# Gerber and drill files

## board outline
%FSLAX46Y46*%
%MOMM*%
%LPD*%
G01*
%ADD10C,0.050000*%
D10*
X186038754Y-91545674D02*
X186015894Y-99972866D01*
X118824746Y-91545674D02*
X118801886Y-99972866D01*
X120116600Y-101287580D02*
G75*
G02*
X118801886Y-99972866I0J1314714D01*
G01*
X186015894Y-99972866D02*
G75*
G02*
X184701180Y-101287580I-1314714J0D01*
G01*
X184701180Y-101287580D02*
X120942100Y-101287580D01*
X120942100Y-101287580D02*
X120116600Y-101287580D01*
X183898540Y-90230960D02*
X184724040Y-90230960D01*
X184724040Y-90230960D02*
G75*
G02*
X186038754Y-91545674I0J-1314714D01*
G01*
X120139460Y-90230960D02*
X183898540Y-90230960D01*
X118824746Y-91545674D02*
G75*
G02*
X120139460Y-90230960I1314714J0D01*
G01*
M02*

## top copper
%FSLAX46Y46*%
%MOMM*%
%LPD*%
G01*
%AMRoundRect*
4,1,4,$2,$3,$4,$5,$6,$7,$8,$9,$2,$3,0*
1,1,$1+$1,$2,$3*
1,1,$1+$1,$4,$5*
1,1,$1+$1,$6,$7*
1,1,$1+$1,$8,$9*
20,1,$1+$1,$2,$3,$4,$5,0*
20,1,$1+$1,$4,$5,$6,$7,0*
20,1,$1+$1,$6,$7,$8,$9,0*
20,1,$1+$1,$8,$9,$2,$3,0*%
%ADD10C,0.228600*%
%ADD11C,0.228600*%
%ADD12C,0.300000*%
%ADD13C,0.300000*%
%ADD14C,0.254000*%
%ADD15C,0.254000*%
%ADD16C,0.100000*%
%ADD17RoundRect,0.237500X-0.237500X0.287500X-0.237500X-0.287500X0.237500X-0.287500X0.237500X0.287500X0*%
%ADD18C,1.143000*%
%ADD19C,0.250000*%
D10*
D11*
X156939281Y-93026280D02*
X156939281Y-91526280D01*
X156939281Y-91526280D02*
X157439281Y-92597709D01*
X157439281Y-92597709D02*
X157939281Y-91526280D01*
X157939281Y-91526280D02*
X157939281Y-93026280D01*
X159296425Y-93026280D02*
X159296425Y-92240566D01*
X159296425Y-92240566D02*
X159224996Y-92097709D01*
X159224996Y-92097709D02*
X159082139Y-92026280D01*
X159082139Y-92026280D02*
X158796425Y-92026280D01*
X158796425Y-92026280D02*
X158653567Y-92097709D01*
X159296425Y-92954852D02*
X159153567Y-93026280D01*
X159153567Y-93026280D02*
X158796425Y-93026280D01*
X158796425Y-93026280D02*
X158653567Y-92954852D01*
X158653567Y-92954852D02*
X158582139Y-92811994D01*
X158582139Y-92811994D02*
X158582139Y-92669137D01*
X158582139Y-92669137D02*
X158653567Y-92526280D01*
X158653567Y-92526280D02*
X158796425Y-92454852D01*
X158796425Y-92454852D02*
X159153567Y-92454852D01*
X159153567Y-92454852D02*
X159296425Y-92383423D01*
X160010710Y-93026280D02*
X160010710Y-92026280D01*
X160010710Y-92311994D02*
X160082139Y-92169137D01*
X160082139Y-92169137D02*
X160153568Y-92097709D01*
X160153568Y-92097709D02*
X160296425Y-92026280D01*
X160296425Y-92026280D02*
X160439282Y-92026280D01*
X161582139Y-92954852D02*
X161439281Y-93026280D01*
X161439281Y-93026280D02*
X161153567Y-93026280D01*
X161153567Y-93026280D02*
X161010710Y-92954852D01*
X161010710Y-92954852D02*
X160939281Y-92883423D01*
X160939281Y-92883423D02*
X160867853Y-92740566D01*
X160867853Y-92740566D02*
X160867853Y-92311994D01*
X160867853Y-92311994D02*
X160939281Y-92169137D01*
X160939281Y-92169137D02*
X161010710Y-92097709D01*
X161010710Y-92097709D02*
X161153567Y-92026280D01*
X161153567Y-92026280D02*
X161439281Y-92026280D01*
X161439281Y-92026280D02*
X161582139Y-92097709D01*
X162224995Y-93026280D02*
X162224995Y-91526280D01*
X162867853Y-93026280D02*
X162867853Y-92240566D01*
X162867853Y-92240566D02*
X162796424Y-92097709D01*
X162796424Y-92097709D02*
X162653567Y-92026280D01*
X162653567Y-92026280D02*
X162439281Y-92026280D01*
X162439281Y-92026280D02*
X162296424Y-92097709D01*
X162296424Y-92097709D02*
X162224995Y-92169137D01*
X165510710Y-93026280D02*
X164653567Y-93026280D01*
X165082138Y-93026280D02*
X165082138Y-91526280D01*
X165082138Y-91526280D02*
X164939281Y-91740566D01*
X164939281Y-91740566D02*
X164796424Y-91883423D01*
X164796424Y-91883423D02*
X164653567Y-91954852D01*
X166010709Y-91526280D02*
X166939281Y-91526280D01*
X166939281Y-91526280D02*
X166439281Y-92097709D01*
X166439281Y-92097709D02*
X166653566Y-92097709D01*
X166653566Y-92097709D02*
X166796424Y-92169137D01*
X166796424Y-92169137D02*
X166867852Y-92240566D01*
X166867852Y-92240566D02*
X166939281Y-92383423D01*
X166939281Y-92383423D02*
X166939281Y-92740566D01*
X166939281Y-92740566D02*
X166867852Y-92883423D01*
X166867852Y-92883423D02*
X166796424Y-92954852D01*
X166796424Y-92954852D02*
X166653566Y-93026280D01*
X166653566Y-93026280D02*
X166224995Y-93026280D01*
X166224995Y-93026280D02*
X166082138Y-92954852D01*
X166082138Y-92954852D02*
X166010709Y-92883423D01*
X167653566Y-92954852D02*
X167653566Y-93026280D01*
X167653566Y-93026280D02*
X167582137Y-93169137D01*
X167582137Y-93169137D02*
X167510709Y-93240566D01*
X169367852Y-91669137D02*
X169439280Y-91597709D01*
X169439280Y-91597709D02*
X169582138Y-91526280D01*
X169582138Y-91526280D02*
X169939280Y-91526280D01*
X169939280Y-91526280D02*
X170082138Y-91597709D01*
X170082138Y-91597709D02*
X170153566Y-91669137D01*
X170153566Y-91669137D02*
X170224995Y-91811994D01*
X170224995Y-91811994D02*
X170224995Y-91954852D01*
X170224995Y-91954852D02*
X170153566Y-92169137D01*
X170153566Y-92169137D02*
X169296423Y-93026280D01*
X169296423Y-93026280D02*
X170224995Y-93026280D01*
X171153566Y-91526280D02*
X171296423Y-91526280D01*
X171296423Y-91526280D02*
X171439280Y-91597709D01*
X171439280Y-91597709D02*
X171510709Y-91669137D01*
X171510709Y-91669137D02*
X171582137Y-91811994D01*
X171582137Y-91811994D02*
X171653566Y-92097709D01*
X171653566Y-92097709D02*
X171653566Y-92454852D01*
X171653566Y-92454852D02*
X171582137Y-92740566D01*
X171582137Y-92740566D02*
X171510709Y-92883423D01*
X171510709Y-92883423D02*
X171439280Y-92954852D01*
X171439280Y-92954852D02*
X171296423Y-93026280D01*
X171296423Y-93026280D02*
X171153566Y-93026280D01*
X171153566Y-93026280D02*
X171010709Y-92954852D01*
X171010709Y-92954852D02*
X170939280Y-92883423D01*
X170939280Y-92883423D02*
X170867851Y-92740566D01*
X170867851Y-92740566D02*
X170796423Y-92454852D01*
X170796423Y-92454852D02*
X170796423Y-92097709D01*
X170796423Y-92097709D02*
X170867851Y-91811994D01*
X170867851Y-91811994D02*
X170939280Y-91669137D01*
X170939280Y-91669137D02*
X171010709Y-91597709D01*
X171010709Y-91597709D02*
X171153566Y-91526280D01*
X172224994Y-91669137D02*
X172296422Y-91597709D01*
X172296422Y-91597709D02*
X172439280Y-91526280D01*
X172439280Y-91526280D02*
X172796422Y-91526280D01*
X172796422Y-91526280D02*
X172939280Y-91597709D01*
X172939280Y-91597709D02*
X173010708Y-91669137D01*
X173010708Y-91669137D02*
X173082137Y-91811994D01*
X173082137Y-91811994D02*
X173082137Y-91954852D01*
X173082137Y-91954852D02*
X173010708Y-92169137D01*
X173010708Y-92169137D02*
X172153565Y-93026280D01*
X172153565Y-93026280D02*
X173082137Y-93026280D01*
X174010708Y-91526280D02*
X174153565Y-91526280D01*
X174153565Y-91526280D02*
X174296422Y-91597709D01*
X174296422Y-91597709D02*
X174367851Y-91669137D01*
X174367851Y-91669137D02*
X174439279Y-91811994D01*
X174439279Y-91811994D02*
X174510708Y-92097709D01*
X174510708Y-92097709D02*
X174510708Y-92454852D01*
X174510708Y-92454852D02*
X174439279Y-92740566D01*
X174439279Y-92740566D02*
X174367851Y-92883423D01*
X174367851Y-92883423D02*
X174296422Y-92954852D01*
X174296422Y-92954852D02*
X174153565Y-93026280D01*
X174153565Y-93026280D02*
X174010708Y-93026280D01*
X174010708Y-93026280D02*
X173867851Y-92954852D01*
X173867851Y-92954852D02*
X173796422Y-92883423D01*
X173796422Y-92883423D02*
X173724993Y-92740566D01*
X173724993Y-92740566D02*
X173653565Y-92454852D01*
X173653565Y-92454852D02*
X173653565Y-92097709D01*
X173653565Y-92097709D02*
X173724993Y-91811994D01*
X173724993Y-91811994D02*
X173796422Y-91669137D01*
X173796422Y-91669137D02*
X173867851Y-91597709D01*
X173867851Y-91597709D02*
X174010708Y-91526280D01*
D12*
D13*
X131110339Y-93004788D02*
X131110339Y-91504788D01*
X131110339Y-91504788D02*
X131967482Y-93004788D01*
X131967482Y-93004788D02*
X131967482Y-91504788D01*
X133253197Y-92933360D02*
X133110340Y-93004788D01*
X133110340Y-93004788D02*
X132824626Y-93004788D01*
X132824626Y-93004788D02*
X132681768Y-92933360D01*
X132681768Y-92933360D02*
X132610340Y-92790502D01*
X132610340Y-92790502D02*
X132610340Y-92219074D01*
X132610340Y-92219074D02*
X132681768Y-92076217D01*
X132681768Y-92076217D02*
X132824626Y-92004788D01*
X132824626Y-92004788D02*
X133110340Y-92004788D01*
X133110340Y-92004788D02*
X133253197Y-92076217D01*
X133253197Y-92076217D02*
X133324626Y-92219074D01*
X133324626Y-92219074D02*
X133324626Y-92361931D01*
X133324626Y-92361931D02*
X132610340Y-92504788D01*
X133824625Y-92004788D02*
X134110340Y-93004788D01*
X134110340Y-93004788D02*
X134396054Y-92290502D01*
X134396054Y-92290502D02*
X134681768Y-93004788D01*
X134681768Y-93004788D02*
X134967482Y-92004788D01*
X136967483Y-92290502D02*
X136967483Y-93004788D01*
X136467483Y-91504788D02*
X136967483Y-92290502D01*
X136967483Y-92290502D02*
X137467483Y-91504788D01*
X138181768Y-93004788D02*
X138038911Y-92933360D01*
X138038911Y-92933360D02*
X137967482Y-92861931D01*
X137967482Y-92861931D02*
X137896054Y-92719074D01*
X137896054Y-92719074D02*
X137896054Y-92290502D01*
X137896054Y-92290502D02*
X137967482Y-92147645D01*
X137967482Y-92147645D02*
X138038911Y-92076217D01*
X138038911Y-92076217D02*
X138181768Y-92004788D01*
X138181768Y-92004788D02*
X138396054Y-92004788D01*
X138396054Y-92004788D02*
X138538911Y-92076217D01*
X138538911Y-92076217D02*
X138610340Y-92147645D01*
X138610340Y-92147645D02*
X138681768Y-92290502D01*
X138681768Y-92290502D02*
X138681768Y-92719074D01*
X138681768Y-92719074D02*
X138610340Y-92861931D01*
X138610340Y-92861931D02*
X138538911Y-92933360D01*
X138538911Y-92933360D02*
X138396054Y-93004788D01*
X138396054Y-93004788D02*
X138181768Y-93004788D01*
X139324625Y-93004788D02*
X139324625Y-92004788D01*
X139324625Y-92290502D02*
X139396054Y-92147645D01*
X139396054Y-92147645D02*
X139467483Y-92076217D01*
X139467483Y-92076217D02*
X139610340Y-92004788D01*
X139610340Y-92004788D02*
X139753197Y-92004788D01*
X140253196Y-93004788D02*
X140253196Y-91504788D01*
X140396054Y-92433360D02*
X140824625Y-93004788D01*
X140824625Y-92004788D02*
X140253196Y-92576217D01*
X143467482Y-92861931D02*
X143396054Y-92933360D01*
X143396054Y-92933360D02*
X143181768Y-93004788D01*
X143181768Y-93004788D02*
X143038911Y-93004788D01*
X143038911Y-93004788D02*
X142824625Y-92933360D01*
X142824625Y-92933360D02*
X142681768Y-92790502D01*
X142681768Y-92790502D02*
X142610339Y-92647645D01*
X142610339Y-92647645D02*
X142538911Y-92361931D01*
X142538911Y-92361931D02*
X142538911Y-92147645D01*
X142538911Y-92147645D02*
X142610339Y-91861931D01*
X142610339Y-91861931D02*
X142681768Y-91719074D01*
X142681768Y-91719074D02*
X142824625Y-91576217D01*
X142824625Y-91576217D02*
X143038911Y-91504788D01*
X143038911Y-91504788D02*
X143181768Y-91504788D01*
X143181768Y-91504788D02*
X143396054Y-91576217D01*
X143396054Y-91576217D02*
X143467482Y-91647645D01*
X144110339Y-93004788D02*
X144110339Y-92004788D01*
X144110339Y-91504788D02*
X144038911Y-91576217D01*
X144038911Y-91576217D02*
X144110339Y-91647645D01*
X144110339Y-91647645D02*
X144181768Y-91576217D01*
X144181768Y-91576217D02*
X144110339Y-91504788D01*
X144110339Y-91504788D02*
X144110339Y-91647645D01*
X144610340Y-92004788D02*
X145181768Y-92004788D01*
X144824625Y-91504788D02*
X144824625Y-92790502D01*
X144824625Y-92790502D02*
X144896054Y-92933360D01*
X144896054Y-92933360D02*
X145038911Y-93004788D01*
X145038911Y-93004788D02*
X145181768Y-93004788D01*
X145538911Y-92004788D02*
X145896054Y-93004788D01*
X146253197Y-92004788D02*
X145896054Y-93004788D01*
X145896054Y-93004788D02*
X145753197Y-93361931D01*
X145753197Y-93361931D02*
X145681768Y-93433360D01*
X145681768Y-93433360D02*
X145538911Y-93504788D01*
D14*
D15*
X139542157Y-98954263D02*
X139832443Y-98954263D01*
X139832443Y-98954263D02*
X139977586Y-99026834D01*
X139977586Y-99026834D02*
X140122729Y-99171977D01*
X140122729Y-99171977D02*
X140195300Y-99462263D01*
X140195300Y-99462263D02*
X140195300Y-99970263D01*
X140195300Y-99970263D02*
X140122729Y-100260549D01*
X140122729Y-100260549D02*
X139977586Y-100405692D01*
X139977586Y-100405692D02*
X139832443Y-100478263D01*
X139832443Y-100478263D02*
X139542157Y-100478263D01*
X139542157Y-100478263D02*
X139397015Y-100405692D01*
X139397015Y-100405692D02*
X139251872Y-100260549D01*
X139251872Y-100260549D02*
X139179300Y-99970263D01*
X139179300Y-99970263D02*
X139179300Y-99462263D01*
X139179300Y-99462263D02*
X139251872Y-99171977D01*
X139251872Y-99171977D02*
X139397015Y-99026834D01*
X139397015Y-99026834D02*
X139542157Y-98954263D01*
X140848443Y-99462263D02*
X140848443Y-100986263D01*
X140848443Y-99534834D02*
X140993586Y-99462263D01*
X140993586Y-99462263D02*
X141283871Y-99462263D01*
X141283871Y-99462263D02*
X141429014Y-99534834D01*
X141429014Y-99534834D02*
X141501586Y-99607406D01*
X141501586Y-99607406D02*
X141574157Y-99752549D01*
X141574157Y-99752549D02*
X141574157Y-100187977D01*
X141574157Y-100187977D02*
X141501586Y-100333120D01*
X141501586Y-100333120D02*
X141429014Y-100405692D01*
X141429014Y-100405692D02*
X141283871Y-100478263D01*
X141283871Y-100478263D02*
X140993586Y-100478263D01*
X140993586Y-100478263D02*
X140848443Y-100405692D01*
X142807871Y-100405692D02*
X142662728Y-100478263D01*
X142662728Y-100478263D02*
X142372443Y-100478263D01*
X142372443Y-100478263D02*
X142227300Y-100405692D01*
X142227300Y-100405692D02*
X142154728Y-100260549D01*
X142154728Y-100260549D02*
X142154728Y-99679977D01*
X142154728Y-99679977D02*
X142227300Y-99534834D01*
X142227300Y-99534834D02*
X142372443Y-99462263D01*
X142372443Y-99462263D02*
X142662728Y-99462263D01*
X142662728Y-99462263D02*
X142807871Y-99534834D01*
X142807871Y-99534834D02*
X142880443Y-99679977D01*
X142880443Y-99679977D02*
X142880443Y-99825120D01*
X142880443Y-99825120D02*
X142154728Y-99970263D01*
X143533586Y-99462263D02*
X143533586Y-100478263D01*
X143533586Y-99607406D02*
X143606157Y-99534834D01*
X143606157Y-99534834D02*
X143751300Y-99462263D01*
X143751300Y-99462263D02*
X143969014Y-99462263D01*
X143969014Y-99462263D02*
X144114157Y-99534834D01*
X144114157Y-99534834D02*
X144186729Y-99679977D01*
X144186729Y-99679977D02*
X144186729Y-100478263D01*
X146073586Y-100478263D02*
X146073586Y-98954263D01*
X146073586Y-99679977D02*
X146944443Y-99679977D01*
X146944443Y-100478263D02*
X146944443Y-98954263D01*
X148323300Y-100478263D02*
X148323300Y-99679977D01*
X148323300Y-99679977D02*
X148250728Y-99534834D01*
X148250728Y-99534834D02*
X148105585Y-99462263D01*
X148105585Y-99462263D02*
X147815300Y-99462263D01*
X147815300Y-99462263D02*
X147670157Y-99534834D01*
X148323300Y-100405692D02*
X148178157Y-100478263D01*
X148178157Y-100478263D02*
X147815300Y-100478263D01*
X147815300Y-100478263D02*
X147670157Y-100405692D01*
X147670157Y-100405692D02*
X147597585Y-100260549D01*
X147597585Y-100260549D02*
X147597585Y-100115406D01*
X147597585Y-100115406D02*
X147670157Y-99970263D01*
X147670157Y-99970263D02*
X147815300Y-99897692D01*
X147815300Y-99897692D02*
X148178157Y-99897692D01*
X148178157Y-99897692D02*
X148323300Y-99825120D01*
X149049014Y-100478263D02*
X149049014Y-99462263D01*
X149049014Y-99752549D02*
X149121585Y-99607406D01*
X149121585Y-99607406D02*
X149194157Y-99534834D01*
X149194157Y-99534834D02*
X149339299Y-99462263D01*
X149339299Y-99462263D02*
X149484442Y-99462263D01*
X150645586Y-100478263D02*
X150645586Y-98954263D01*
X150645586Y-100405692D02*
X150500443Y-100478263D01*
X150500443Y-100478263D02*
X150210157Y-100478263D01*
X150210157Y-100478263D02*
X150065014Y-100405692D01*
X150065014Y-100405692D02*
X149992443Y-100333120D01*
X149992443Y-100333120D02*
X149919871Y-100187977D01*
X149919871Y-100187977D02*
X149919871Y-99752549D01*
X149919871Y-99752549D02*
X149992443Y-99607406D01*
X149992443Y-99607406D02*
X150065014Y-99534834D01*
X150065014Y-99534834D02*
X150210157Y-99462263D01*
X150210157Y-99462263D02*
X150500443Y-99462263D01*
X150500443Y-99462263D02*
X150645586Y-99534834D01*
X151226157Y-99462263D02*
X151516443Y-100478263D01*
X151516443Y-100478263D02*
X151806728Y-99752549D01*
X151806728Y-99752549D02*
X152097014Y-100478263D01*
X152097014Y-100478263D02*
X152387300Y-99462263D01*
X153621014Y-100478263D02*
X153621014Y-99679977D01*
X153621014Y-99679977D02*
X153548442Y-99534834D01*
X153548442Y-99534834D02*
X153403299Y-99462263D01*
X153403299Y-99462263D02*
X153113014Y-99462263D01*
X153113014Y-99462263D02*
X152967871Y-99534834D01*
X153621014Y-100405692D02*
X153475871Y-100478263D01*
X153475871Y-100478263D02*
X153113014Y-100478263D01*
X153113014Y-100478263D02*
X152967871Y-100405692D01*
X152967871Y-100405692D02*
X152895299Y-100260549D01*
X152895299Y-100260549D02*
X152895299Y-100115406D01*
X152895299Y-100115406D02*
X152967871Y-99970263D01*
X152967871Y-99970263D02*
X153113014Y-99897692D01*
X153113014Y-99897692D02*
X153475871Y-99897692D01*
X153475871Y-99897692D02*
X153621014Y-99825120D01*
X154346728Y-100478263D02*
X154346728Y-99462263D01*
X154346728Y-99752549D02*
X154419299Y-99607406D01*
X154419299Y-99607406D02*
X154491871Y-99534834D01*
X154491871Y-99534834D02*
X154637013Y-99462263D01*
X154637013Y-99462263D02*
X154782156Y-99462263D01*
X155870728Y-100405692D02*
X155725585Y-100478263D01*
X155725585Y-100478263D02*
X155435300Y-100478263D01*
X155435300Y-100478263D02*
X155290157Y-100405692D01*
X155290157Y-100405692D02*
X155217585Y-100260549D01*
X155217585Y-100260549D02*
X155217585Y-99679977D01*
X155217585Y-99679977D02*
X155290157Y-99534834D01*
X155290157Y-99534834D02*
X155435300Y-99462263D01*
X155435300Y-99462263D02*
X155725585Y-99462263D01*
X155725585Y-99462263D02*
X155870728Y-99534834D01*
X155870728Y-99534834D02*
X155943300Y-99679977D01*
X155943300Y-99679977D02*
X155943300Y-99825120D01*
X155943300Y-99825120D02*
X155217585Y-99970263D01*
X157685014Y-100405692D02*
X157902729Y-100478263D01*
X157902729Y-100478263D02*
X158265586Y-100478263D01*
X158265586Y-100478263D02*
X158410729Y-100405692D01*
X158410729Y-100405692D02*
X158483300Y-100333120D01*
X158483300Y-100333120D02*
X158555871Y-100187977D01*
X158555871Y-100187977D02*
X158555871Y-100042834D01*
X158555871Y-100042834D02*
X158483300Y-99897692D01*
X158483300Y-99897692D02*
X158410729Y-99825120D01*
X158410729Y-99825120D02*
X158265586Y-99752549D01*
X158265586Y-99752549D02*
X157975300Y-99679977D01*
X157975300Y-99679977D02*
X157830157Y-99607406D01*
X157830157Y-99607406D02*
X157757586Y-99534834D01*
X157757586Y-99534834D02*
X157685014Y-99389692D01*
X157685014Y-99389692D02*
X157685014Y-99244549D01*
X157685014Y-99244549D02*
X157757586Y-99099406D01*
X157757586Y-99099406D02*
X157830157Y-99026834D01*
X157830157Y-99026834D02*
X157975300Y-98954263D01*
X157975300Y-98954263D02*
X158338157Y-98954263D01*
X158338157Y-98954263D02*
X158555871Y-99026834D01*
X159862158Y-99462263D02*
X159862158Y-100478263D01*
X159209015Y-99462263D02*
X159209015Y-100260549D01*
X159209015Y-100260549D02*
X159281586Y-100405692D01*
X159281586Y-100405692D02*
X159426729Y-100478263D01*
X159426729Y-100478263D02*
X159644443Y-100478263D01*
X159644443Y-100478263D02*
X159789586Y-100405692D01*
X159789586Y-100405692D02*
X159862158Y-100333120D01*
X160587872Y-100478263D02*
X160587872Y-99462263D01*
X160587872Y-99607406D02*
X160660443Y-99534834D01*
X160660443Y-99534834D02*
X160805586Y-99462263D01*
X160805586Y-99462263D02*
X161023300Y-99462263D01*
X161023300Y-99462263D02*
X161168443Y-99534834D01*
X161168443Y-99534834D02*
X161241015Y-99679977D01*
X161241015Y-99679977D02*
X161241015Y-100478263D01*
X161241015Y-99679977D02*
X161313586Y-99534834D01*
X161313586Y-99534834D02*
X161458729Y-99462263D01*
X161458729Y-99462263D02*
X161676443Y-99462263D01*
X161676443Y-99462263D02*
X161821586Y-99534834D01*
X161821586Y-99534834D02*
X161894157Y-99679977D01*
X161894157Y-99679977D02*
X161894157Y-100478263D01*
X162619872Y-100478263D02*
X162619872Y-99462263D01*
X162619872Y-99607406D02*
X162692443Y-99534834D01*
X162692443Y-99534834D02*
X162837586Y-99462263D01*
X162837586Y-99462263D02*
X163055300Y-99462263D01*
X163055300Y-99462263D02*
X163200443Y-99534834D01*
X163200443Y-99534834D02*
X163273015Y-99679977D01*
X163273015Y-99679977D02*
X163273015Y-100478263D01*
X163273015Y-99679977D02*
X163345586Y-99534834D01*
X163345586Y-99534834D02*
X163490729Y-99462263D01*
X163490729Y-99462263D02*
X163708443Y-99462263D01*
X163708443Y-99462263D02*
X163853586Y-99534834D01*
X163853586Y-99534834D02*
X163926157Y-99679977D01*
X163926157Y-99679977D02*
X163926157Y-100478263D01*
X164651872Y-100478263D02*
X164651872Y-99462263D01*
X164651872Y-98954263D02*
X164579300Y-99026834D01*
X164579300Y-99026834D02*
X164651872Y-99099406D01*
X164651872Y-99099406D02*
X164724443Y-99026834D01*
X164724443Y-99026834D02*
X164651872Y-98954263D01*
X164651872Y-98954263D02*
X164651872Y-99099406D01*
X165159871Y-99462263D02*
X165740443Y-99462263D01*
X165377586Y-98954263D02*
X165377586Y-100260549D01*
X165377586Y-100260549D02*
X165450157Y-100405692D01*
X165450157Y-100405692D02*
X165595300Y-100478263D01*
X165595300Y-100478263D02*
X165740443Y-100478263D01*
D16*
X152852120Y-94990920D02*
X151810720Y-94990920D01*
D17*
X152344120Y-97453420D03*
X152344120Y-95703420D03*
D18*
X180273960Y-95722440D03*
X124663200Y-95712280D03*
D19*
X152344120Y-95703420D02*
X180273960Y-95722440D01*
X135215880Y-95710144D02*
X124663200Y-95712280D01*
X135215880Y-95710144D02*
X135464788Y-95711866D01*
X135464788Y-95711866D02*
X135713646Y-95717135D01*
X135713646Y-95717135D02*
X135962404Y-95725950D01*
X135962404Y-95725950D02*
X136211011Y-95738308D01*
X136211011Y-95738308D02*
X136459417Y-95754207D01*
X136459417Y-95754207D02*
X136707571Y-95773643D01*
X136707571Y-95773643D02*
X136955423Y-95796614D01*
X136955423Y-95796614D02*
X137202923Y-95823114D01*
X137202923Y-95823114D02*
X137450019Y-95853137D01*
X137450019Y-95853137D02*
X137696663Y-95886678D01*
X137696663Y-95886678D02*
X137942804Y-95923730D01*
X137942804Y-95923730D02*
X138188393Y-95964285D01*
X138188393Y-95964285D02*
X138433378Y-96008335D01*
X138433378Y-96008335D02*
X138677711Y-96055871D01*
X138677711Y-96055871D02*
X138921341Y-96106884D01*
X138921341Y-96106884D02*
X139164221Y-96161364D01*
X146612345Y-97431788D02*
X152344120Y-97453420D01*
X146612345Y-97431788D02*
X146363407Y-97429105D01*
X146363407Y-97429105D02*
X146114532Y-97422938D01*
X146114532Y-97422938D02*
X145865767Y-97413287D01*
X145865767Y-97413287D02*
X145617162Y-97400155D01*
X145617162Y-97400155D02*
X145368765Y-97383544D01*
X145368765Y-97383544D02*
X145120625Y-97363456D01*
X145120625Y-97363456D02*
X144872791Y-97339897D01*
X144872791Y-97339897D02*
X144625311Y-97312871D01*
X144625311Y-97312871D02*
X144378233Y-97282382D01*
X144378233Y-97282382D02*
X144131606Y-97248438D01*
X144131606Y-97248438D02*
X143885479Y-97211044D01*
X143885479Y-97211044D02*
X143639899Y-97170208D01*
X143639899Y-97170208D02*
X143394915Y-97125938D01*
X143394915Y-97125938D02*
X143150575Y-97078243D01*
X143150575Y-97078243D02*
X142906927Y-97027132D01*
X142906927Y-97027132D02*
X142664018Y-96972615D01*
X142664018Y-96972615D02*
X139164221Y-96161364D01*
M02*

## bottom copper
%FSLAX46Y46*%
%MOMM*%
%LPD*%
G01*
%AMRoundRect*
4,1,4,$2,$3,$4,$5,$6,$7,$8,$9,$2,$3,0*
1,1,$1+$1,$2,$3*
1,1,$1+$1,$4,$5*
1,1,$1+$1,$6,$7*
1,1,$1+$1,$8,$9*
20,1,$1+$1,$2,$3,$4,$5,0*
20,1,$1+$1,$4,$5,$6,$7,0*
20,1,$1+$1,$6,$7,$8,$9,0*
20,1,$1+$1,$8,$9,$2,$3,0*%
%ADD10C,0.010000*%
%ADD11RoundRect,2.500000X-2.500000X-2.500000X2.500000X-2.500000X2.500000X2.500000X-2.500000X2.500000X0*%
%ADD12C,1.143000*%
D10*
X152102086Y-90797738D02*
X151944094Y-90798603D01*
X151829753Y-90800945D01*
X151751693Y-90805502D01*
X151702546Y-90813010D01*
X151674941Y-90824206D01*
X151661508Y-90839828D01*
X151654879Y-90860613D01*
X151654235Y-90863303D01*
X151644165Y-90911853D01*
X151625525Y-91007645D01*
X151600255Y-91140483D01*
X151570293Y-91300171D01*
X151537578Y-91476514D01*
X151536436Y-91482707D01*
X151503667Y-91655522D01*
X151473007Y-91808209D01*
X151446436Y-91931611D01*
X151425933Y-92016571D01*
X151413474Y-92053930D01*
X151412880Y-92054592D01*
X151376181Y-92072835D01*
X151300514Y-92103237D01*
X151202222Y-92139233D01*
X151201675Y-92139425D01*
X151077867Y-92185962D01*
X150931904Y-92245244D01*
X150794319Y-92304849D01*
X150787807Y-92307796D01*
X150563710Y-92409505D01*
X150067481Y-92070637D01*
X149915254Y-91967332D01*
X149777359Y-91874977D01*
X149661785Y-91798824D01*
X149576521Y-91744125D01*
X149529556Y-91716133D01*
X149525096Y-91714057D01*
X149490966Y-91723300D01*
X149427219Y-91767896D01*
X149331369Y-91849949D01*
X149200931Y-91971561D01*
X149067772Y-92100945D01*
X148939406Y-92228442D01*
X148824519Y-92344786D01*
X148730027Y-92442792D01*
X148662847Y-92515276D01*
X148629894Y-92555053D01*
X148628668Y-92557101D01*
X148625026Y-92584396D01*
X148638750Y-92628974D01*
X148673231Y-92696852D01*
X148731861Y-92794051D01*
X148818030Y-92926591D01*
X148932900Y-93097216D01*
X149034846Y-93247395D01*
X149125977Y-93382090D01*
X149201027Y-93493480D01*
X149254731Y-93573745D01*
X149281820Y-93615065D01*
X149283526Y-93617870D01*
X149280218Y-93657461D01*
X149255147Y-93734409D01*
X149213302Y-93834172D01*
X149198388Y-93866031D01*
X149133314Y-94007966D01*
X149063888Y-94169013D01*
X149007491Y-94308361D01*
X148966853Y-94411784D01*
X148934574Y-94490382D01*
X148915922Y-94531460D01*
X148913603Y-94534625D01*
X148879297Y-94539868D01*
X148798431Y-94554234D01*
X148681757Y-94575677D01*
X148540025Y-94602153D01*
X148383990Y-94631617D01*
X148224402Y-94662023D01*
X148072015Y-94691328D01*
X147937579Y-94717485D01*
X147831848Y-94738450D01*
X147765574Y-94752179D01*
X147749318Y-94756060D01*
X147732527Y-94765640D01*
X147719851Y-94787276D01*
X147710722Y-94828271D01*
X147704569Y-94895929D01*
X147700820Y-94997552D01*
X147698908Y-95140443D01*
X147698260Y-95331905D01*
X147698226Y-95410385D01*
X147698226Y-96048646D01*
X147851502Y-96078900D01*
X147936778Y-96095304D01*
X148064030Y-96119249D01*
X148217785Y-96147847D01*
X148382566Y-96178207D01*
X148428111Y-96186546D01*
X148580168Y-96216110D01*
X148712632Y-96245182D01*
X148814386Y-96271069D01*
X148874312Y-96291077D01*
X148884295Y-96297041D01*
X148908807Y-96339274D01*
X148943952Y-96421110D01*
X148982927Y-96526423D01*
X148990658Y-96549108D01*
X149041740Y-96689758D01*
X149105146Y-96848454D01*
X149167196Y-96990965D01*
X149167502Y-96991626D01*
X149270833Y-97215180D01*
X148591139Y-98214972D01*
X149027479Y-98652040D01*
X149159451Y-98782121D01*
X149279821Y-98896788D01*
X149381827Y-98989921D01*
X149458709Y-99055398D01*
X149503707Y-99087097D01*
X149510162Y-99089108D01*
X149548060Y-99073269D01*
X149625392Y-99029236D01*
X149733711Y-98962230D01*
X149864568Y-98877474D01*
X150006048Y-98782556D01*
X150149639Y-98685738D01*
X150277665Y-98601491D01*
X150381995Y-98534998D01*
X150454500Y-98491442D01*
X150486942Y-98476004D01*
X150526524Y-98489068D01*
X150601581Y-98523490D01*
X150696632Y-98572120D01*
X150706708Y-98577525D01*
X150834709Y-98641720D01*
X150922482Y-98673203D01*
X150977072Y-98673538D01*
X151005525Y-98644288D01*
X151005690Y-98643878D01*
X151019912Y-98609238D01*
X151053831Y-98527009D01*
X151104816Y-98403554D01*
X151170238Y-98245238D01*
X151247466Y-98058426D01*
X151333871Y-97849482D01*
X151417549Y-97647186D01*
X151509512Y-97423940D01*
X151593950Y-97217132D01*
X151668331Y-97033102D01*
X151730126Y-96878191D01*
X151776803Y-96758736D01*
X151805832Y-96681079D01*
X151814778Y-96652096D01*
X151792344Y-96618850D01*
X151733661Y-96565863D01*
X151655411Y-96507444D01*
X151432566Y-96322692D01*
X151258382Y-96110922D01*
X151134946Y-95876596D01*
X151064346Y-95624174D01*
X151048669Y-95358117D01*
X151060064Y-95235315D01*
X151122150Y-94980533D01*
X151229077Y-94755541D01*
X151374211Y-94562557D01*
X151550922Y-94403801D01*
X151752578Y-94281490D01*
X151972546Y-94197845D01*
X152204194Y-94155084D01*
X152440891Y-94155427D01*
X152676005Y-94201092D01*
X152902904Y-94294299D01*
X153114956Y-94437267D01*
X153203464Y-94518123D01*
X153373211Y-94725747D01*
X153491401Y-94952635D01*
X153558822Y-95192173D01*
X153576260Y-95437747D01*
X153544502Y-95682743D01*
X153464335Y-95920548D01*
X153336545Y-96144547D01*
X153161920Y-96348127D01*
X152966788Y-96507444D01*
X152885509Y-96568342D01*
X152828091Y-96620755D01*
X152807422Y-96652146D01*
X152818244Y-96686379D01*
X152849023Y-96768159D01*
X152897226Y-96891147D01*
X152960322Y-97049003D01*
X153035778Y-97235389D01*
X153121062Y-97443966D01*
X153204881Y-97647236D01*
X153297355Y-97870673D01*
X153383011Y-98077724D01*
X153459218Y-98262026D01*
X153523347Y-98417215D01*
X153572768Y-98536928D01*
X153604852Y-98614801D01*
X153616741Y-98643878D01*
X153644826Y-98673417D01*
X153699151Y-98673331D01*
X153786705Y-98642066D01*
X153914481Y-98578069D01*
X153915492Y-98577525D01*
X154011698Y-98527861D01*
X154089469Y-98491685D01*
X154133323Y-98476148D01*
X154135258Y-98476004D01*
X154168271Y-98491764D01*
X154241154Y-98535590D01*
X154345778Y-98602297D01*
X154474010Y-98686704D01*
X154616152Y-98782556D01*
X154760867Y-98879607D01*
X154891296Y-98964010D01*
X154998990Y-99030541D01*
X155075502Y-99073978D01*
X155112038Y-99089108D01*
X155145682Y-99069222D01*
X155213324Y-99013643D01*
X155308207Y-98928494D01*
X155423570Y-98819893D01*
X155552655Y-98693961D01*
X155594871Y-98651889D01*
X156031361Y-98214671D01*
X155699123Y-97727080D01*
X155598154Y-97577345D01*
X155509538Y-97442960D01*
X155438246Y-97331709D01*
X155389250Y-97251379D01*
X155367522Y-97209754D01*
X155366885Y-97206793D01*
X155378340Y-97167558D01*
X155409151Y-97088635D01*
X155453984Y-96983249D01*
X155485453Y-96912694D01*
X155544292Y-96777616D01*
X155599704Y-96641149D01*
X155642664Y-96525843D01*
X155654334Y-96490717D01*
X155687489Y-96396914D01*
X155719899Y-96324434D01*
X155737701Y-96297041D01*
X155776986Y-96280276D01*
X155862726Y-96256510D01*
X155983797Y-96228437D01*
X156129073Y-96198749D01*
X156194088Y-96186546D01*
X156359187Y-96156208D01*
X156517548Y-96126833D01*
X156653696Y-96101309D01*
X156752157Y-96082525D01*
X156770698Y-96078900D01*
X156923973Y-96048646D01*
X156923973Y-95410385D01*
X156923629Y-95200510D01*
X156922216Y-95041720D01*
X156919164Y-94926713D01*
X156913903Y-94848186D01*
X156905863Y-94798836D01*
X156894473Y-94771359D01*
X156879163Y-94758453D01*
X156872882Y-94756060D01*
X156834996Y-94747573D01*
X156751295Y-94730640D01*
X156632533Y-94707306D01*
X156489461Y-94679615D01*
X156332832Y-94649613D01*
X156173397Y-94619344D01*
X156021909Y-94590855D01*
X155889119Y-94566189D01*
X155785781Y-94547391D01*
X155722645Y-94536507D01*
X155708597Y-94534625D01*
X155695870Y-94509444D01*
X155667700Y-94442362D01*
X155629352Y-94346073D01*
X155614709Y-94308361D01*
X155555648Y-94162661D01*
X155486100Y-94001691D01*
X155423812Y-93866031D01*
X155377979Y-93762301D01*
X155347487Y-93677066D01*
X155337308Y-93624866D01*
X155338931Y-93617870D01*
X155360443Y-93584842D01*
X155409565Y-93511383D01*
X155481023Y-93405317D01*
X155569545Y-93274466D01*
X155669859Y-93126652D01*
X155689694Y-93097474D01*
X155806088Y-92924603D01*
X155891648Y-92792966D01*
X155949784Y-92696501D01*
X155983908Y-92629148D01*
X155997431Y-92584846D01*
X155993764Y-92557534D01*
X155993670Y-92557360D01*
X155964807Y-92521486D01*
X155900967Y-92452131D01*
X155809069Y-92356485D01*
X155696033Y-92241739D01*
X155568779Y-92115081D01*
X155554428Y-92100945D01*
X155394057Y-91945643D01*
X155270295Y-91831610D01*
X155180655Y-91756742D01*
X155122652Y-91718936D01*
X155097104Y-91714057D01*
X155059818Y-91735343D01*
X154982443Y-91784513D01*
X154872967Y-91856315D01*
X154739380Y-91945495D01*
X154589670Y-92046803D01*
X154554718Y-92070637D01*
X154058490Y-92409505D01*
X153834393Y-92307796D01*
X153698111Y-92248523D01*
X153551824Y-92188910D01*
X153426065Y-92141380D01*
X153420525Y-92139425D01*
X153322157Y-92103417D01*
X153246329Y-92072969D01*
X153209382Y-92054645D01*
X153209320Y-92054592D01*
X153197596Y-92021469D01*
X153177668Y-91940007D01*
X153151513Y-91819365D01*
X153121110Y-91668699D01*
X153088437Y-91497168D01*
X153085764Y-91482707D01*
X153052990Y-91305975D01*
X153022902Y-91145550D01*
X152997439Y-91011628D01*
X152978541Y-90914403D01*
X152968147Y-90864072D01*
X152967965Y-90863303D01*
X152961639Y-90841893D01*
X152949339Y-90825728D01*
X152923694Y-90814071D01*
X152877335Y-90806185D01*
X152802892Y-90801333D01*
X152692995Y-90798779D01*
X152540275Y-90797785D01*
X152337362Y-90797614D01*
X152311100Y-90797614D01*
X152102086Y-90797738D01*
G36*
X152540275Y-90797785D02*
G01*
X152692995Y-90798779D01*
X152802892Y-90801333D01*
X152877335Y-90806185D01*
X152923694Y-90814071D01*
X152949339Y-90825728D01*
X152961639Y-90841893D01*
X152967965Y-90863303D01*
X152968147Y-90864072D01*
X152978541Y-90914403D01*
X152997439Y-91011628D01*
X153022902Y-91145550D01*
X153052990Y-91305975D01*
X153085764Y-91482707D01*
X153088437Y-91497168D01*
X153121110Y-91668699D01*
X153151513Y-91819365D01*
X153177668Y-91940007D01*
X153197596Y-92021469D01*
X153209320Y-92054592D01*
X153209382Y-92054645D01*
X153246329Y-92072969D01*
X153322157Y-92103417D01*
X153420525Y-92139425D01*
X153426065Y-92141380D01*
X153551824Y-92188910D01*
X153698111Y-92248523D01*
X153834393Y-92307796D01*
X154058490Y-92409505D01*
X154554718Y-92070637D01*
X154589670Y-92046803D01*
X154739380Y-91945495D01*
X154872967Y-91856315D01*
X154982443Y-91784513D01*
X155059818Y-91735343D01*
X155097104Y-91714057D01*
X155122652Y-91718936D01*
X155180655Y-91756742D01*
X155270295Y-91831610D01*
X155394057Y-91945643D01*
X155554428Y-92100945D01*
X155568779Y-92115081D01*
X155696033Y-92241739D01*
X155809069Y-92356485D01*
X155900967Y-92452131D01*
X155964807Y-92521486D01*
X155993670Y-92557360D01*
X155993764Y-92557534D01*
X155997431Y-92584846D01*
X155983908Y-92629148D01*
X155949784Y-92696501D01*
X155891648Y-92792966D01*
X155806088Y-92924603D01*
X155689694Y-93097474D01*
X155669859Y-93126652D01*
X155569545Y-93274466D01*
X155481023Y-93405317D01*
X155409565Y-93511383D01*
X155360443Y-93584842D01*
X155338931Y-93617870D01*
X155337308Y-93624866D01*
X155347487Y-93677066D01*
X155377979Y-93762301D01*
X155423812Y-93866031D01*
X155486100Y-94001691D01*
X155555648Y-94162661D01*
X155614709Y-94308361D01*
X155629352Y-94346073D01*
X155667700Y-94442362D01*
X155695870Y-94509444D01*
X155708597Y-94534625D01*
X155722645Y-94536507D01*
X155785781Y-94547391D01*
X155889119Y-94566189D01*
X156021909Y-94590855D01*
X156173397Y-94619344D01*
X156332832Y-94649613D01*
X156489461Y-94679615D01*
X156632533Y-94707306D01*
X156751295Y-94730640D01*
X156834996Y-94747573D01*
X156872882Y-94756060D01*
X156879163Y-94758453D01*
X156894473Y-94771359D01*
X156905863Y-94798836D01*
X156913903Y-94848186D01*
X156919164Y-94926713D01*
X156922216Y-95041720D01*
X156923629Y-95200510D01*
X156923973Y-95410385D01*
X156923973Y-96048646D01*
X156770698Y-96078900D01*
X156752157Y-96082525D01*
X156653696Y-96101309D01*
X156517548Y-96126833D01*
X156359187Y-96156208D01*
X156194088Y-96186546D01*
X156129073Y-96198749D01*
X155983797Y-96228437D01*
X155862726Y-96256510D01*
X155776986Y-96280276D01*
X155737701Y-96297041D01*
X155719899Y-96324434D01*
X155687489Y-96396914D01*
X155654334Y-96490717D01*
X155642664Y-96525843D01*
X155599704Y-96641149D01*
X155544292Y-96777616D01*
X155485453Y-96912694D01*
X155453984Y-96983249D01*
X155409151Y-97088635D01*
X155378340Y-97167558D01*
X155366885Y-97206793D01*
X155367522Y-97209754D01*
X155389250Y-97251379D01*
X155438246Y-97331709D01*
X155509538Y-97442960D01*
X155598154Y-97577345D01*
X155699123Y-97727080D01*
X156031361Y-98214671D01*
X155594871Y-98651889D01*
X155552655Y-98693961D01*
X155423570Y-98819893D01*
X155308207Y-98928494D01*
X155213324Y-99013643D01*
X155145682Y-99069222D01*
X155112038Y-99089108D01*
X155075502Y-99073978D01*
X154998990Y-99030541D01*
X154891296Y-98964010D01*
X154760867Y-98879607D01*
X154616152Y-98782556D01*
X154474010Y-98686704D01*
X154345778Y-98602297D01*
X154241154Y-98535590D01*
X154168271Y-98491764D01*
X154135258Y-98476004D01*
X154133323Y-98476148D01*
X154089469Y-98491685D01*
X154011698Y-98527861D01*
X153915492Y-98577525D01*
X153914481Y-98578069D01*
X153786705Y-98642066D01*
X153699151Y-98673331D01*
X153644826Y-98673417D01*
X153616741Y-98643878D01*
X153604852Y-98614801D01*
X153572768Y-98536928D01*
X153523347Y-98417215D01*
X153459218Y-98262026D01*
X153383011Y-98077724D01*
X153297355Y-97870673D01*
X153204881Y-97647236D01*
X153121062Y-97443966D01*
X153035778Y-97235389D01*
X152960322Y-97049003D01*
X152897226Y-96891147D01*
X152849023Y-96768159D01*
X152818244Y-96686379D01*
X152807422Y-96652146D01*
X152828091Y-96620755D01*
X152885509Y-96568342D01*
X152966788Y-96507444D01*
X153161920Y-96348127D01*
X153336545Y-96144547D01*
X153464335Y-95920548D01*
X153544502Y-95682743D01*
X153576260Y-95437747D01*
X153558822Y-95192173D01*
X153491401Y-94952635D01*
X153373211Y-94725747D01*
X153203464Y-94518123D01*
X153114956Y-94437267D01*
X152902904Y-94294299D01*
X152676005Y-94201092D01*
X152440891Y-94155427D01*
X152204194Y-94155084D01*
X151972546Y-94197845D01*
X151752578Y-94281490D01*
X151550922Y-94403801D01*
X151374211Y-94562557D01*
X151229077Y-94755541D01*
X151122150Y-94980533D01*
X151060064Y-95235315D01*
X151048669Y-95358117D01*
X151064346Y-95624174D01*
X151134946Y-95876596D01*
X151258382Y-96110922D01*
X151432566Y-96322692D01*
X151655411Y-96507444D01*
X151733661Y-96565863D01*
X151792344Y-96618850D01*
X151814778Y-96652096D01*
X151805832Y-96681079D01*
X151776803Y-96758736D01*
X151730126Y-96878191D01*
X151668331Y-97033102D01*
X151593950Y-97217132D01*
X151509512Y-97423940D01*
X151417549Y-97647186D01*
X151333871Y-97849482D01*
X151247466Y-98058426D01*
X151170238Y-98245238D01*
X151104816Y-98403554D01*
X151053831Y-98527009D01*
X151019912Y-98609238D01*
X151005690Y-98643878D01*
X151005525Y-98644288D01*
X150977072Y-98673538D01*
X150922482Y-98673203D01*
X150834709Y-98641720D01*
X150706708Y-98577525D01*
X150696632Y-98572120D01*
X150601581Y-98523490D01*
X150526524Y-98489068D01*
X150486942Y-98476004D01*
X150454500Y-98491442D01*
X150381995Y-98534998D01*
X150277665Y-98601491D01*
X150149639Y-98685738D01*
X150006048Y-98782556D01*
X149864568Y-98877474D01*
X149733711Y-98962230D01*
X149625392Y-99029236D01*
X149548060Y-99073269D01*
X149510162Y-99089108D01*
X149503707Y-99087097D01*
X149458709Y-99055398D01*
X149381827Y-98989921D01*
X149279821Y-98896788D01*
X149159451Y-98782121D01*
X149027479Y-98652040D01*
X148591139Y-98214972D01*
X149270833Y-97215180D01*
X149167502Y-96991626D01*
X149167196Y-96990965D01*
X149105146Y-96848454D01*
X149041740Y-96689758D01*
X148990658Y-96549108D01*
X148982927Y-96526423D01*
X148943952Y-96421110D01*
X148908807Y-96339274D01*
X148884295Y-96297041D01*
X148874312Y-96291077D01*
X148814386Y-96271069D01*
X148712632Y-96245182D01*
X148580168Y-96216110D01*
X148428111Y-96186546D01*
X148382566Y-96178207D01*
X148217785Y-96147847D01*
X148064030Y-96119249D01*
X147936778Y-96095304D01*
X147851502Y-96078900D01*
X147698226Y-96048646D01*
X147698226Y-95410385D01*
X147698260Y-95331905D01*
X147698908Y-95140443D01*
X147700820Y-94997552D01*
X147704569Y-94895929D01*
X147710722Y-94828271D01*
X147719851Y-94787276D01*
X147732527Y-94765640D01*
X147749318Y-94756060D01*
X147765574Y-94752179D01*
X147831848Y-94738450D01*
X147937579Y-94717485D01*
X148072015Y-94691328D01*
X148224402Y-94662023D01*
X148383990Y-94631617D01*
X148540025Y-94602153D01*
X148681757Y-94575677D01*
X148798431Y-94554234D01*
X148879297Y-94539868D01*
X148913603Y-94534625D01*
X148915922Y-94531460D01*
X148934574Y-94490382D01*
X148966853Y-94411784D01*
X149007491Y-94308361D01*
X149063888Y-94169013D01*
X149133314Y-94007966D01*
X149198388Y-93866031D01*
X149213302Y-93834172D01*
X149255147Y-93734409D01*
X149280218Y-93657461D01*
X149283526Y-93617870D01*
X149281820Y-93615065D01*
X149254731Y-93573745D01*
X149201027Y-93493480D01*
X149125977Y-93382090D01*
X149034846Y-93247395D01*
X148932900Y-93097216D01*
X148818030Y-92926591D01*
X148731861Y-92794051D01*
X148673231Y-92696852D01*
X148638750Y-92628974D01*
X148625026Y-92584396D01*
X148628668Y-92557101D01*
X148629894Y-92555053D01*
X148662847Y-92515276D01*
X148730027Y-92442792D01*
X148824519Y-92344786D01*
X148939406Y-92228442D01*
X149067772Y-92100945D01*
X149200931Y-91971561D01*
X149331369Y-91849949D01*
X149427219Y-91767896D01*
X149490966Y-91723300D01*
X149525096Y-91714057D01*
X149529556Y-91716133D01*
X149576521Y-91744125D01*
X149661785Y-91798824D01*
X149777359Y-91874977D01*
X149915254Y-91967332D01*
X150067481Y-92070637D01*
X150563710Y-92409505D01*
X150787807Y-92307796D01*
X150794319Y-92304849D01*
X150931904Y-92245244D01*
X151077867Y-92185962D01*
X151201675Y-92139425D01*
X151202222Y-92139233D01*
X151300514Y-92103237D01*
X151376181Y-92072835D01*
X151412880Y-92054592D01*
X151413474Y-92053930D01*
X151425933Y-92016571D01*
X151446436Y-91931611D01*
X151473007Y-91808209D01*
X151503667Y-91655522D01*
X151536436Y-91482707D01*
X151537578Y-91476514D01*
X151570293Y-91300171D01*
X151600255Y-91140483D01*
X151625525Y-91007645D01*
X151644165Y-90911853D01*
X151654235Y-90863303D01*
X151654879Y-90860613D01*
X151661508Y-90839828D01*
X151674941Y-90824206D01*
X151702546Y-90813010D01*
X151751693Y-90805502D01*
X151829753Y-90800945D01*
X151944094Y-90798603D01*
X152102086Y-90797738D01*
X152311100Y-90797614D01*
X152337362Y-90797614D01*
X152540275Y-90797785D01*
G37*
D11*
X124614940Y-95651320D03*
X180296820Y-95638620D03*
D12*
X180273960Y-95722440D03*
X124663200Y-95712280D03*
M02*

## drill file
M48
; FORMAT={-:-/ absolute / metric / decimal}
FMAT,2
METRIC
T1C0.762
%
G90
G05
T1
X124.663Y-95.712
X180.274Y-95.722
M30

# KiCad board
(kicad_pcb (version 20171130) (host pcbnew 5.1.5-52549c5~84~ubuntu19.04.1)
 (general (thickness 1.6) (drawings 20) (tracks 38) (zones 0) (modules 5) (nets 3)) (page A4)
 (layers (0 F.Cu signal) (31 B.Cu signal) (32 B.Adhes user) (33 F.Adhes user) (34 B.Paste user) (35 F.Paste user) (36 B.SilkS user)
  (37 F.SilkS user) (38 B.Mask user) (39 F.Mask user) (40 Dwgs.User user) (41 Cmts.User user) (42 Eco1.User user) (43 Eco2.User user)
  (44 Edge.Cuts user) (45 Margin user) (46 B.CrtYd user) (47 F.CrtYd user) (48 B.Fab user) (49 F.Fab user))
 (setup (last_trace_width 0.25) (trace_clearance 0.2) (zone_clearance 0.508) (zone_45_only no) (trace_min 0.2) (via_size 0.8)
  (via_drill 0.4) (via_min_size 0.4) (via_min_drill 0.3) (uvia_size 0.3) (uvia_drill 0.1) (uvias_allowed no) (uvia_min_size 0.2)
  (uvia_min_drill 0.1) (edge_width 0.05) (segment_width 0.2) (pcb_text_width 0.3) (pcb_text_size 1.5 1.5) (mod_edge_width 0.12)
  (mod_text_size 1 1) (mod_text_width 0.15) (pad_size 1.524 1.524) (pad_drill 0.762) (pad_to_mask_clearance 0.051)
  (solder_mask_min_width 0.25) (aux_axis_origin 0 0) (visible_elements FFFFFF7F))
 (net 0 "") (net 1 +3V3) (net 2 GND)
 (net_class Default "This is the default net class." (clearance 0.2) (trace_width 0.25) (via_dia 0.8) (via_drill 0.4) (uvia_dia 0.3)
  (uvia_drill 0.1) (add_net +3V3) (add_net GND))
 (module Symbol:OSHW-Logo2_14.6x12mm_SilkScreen (layer B.Cu) (at 152.3111 96.34474 180)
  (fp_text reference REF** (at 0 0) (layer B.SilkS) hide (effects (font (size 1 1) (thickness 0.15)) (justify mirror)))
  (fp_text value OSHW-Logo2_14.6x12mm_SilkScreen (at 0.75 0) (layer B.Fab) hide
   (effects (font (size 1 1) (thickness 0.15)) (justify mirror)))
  (fp_poly
   (pts (xy 0.209014 5.547002) (xy 0.367006 5.546137) (xy 0.481347 5.543795) (xy 0.559407 5.539238) (xy 0.608554 5.53173)
    (xy 0.636159 5.520534) (xy 0.649592 5.504912) (xy 0.656221 5.484127) (xy 0.656865 5.481437) (xy 0.666935 5.432887)
    (xy 0.685575 5.337095) (xy 0.710845 5.204257) (xy 0.740807 5.044569) (xy 0.773522 4.868226) (xy 0.774664 4.862033)
    (xy 0.807433 4.689218) (xy 0.838093 4.536531) (xy 0.864664 4.413129) (xy 0.885167 4.328169) (xy 0.897626 4.29081) (xy 0.89822 4.290148)
    (xy 0.934919 4.271905) (xy 1.010586 4.241503) (xy 1.108878 4.205507) (xy 1.109425 4.205315) (xy 1.233233 4.158778)
    (xy 1.379196 4.099496) (xy 1.516781 4.039891) (xy 1.523293 4.036944) (xy 1.74739 3.935235) (xy 2.243619 4.274103) (xy 2.395846 4.377408)
    (xy 2.533741 4.469763) (xy 2.649315 4.545916) (xy 2.734579 4.600615) (xy 2.781544 4.628607) (xy 2.786004 4.630683) (xy 2.820134 4.62144)
    (xy 2.883881 4.576844) (xy 2.979731 4.494791) (xy 3.110169 4.373179) (xy 3.243328 4.243795) (xy 3.371694 4.116298)
    (xy 3.486581 3.999954) (xy 3.581073 3.901948) (xy 3.648253 3.829464) (xy 3.681206 3.789687) (xy 3.682432 3.787639)
    (xy 3.686074 3.760344) (xy 3.67235 3.715766) (xy 3.637869 3.647888) (xy 3.579239 3.550689) (xy 3.49307 3.418149) (xy 3.3782 3.247524)
    (xy 3.276254 3.097345) (xy 3.185123 2.96265) (xy 3.110073 2.85126) (xy 3.056369 2.770995) (xy 3.02928 2.729675) (xy 3.027574 2.72687)
    (xy 3.030882 2.687279) (xy 3.055953 2.610331) (xy 3.097798 2.510568) (xy 3.112712 2.478709) (xy 3.177786 2.336774)
    (xy 3.247212 2.175727) (xy 3.303609 2.036379) (xy 3.344247 1.932956) (xy 3.376526 1.854358) (xy 3.395178 1.81328) (xy 3.397497 1.810115)
    (xy 3.431803 1.804872) (xy 3.512669 1.790506) (xy 3.629343 1.769063) (xy 3.771075 1.742587) (xy 3.92711 1.713123) (xy 4.086698 1.682717)
    (xy 4.239085 1.653412) (xy 4.373521 1.627255) (xy 4.479252 1.60629) (xy 4.545526 1.592561) (xy 4.561782 1.58868) (xy 4.578573 1.5791)
    (xy 4.591249 1.557464) (xy 4.600378 1.516469) (xy 4.606531 1.448811) (xy 4.61028 1.347188) (xy 4.612192 1.204297) (xy 4.61284 1.012835)
    (xy 4.612874 0.934355) (xy 4.612874 0.296094) (xy 4.459598 0.26584) (xy 4.374322 0.249436) (xy 4.24707 0.225491) (xy 4.093315 0.196893)
    (xy 3.928534 0.166533) (xy 3.882989 0.158194) (xy 3.730932 0.12863) (xy 3.598468 0.099558) (xy 3.496714 0.073671) (xy 3.436788 0.053663)
    (xy 3.426805 0.047699) (xy 3.402293 0.005466) (xy 3.367148 -0.07637) (xy 3.328173 -0.181683) (xy 3.320442 -0.204368)
    (xy 3.26936 -0.345018) (xy 3.205954 -0.503714) (xy 3.143904 -0.646225) (xy 3.143598 -0.646886) (xy 3.040267 -0.87044)
    (xy 3.719961 -1.870232) (xy 3.283621 -2.3073) (xy 3.151649 -2.437381) (xy 3.031279 -2.552048) (xy 2.929273 -2.645181)
    (xy 2.852391 -2.710658) (xy 2.807393 -2.742357) (xy 2.800938 -2.744368) (xy 2.76304 -2.728529) (xy 2.685708 -2.684496)
    (xy 2.577389 -2.61749) (xy 2.446532 -2.532734) (xy 2.305052 -2.437816) (xy 2.161461 -2.340998) (xy 2.033435 -2.256751)
    (xy 1.929105 -2.190258) (xy 1.8566 -2.146702) (xy 1.824158 -2.131264) (xy 1.784576 -2.144328) (xy 1.709519 -2.17875)
    (xy 1.614468 -2.22738) (xy 1.604392 -2.232785) (xy 1.476391 -2.29698) (xy 1.388618 -2.328463) (xy 1.334028 -2.328798)
    (xy 1.305575 -2.299548) (xy 1.30541 -2.299138) (xy 1.291188 -2.264498) (xy 1.257269 -2.182269) (xy 1.206284 -2.058814)
    (xy 1.140862 -1.900498) (xy 1.063634 -1.713686) (xy 0.977229 -1.504742) (xy 0.893551 -1.302446) (xy 0.801588 -1.0792)
    (xy 0.71715 -0.872392) (xy 0.642769 -0.688362) (xy 0.580974 -0.533451) (xy 0.534297 -0.413996) (xy 0.505268 -0.336339)
    (xy 0.496322 -0.307356) (xy 0.518756 -0.27411) (xy 0.577439 -0.221123) (xy 0.655689 -0.162704) (xy 0.878534 0.022048)
    (xy 1.052718 0.233818) (xy 1.176154 0.468144) (xy 1.246754 0.720566) (xy 1.262431 0.986623) (xy 1.251036 1.109425) (xy 1.18895 1.364207)
    (xy 1.082023 1.589199) (xy 0.936889 1.782183) (xy 0.760178 1.940939) (xy 0.558522 2.06325) (xy 0.338554 2.146895) (xy 0.106906 2.189656)
    (xy -0.129791 2.189313) (xy -0.364905 2.143648) (xy -0.591804 2.050441) (xy -0.803856 1.907473) (xy -0.892364 1.826617)
    (xy -1.062111 1.618993) (xy -1.180301 1.392105) (xy -1.247722 1.152567) (xy -1.26516 0.906993) (xy -1.233402 0.661997)
    (xy -1.153235 0.424192) (xy -1.025445 0.200193) (xy -0.85082 -0.003387) (xy -0.655688 -0.162704) (xy -0.574409 -0.223602)
    (xy -0.516991 -0.276015) (xy -0.496322 -0.307406) (xy -0.507144 -0.341639) (xy -0.537923 -0.423419) (xy -0.586126 -0.546407)
    (xy -0.649222 -0.704263) (xy -0.724678 -0.890649) (xy -0.809962 -1.099226) (xy -0.893781 -1.302496) (xy -0.986255 -1.525933)
    (xy -1.071911 -1.732984) (xy -1.148118 -1.917286) (xy -1.212247 -2.072475) (xy -1.261668 -2.192188) (xy -1.293752 -2.270061)
    (xy -1.305641 -2.299138) (xy -1.333726 -2.328677) (xy -1.388051 -2.328591) (xy -1.475605 -2.297326) (xy -1.603381 -2.233329)
    (xy -1.604392 -2.232785) (xy -1.700598 -2.183121) (xy -1.778369 -2.146945) (xy -1.822223 -2.131408) (xy -1.824158 -2.131264)
    (xy -1.857171 -2.147024) (xy -1.930054 -2.19085) (xy -2.034678 -2.257557) (xy -2.16291 -2.341964) (xy -2.305052 -2.437816)
    (xy -2.449767 -2.534867) (xy -2.580196 -2.61927) (xy -2.68789 -2.685801) (xy -2.764402 -2.729238) (xy -2.800938 -2.744368)
    (xy -2.834582 -2.724482) (xy -2.902224 -2.668903) (xy -2.997107 -2.583754) (xy -3.11247 -2.475153) (xy -3.241555 -2.349221)
    (xy -3.283771 -2.307149) (xy -3.720261 -1.869931) (xy -3.388023 -1.38234) (xy -3.287054 -1.232605) (xy -3.198438 -1.09822)
    (xy -3.127146 -0.986969) (xy -3.07815 -0.906639) (xy -3.056422 -0.865014) (xy -3.055785 -0.862053) (xy -3.06724 -0.822818)
    (xy -3.098051 -0.743895) (xy -3.142884 -0.638509) (xy -3.174353 -0.567954) (xy -3.233192 -0.432876) (xy -3.288604 -0.296409)
    (xy -3.331564 -0.181103) (xy -3.343234 -0.145977) (xy -3.376389 -0.052174) (xy -3.408799 0.020306) (xy -3.426601 0.047699)
    (xy -3.465886 0.064464) (xy -3.551626 0.08823) (xy -3.672697 0.116303) (xy -3.817973 0.145991) (xy -3.882988 0.158194)
    (xy -4.048087 0.188532) (xy -4.206448 0.217907) (xy -4.342596 0.243431) (xy -4.441057 0.262215) (xy -4.459598 0.26584)
    (xy -4.612873 0.296094) (xy -4.612873 0.934355) (xy -4.612529 1.14423) (xy -4.611116 1.30302) (xy -4.608064 1.418027)
    (xy -4.602803 1.496554) (xy -4.594763 1.545904) (xy -4.583373 1.573381) (xy -4.568063 1.586287) (xy -4.561782 1.58868)
    (xy -4.523896 1.597167) (xy -4.440195 1.6141) (xy -4.321433 1.637434) (xy -4.178361 1.665125) (xy -4.021732 1.695127)
    (xy -3.862297 1.725396) (xy -3.710809 1.753885) (xy -3.578019 1.778551) (xy -3.474681 1.797349) (xy -3.411545 1.808233)
    (xy -3.397497 1.810115) (xy -3.38477 1.835296) (xy -3.3566 1.902378) (xy -3.318252 1.998667) (xy -3.303609 2.036379)
    (xy -3.244548 2.182079) (xy -3.175 2.343049) (xy -3.112712 2.478709) (xy -3.066879 2.582439) (xy -3.036387 2.667674)
    (xy -3.026208 2.719874) (xy -3.027831 2.72687) (xy -3.049343 2.759898) (xy -3.098465 2.833357) (xy -3.169923 2.939423)
    (xy -3.258445 3.070274) (xy -3.358759 3.218088) (xy -3.378594 3.247266) (xy -3.494988 3.420137) (xy -3.580548 3.551774)
    (xy -3.638684 3.648239) (xy -3.672808 3.715592) (xy -3.686331 3.759894) (xy -3.682664 3.787206) (xy -3.68257 3.78738)
    (xy -3.653707 3.823254) (xy -3.589867 3.892609) (xy -3.497969 3.988255) (xy -3.384933 4.103001) (xy -3.257679 4.229659)
    (xy -3.243328 4.243795) (xy -3.082957 4.399097) (xy -2.959195 4.51313) (xy -2.869555 4.587998) (xy -2.811552 4.625804)
    (xy -2.786004 4.630683) (xy -2.748718 4.609397) (xy -2.671343 4.560227) (xy -2.561867 4.488425) (xy -2.42828 4.399245)
    (xy -2.27857 4.297937) (xy -2.243618 4.274103) (xy -1.74739 3.935235) (xy -1.523293 4.036944) (xy -1.387011 4.096217)
    (xy -1.240724 4.15583) (xy -1.114965 4.20336) (xy -1.109425 4.205315) (xy -1.011057 4.241323) (xy -0.935229 4.271771)
    (xy -0.898282 4.290095) (xy -0.89822 4.290148) (xy -0.886496 4.323271) (xy -0.866568 4.404733) (xy -0.840413 4.525375)
    (xy -0.81001 4.676041) (xy -0.777337 4.847572) (xy -0.774664 4.862033) (xy -0.74189 5.038765) (xy -0.711802 5.19919)
    (xy -0.686339 5.333112) (xy -0.667441 5.430337) (xy -0.657047 5.480668) (xy -0.656865 5.481437) (xy -0.650539 5.502847)
    (xy -0.638239 5.519012) (xy -0.612594 5.530669) (xy -0.566235 5.538555) (xy -0.491792 5.543407) (xy -0.381895 5.545961)
    (xy -0.229175 5.546955) (xy -0.026262 5.547126) (xy 0 5.547126) (xy 0.209014 5.547002))
   (layer B.Cu) (width 0.01)))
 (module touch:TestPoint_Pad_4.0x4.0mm (layer B.Cu) (at 124.61494 95.65132)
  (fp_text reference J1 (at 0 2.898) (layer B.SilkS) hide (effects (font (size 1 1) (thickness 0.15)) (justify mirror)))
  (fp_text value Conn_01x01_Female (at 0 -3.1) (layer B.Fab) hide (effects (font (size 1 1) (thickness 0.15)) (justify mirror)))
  (pad 1 smd roundrect (at 0 0) (size 10 10) (layers B.Cu B.Mask) (roundrect_rratio 0.25) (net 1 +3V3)))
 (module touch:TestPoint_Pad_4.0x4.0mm (layer B.Cu) (at 180.29682 95.63862)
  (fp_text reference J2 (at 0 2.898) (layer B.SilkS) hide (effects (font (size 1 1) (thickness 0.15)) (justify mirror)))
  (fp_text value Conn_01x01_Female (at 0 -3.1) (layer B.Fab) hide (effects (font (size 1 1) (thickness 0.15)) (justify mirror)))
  (pad 1 smd roundrect (at 0 0) (size 10 10) (layers B.Cu B.Mask) (roundrect_rratio 0.25) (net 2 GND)))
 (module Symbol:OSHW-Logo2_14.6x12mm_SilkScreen (layer F.Cu) (at 152.31364 96.33204)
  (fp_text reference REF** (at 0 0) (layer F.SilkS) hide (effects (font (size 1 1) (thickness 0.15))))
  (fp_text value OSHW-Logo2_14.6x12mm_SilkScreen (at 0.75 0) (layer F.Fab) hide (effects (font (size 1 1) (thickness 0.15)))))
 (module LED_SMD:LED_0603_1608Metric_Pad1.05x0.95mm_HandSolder (layer F.Cu) (at 152.34412 96.57842 270)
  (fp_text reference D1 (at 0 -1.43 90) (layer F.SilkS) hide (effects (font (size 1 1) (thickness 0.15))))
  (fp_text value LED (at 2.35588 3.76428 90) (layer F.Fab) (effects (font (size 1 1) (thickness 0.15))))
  (fp_line (start -1.5875 -0.508) (end -1.5875 0.5334) (layer F.Cu) (width 0.1))
  (pad 2 smd roundrect (at 0.875 0 270) (size 1.05 0.95) (layers F.Cu F.Paste F.Mask) (roundrect_rratio 0.25) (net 1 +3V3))
  (pad 1 smd roundrect (at -0.875 0 270) (size 1.05 0.95) (layers F.Cu F.Paste F.Mask) (roundrect_rratio 0.25) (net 2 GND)))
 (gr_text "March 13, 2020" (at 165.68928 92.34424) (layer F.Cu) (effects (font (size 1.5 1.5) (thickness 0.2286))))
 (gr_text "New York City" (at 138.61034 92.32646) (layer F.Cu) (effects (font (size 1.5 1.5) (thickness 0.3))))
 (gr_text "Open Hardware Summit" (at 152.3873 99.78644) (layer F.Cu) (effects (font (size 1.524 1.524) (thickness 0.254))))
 (gr_line (start 186.038754 91.545674) (end 186.015894 99.972866) (layer Edge.Cuts) (width 0.05))
 (gr_line (start 118.824746 91.545674) (end 118.801886 99.972866) (layer Edge.Cuts) (width 0.05))
 (gr_arc (start 120.1166 99.972866) (end 120.1166 101.28758) (angle 90) (layer Edge.Cuts) (width 0.05))
 (gr_arc (start 184.70118 99.972866) (end 184.70118 101.28758) (angle -90) (layer Edge.Cuts) (width 0.05))
 (gr_line (start 184.70118 101.28758) (end 120.9421 101.28758) (layer Edge.Cuts) (width 0.05))
 (gr_line (start 120.9421 101.28758) (end 120.1166 101.28758) (layer Edge.Cuts) (width 0.05))
 (gr_line (start 183.89854 90.23096) (end 184.72404 90.23096) (layer Edge.Cuts) (width 0.05))
 (gr_arc (start 184.72404 91.545674) (end 184.72404 90.23096) (angle 90) (layer Edge.Cuts) (width 0.05))
 (gr_line (start 120.13946 90.23096) (end 183.89854 90.23096) (layer Edge.Cuts) (width 0.05))
 (gr_arc (start 120.13946 91.545674) (end 120.13946 90.23096) (angle -90) (layer Edge.Cuts) (width 0.05))
 (via (at 180.27396 95.72244) (size 1.143) (drill 0.762) (layers F.Cu B.Cu) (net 2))
 (via (at 124.6632 95.71228) (size 1.143) (drill 0.762) (layers F.Cu B.Cu) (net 1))
 (segment (start 152.34412 95.70342) (end 180.27396 95.72244) (width 0.25) (layer F.Cu) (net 2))
 (segment (start 135.21588 95.710144) (end 124.6632 95.71228) (width 0.25) (layer F.Cu) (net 1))
 (segment (start 135.21588 95.710144) (end 135.464788 95.711866) (width 0.25) (layer F.Cu) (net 1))
 (segment (start 135.464788 95.711866) (end 135.713646 95.717135) (width 0.25) (layer F.Cu) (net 1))
 (segment (start 135.713646 95.717135) (end 135.962404 95.72595) (width 0.25) (layer F.Cu) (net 1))
 (segment (start 135.962404 95.72595) (end 136.211011 95.738308) (width 0.25) (layer F.Cu) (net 1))
 (segment (start 136.211011 95.738308) (end 136.459417 95.754207) (width 0.25) (layer F.Cu) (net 1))
 (segment (start 136.459417 95.754207) (end 136.707571 95.773643) (width 0.25) (layer F.Cu) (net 1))
 (segment (start 136.707571 95.773643) (end 136.955423 95.796614) (width 0.25) (layer F.Cu) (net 1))
 (segment (start 136.955423 95.796614) (end 137.202923 95.823114) (width 0.25) (layer F.Cu) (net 1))
 (segment (start 137.202923 95.823114) (end 137.450019 95.853137) (width 0.25) (layer F.Cu) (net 1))
 (segment (start 137.450019 95.853137) (end 137.696663 95.886678) (width 0.25) (layer F.Cu) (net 1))
 (segment (start 137.696663 95.886678) (end 137.942804 95.92373) (width 0.25) (layer F.Cu) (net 1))
 (segment (start 137.942804 95.92373) (end 138.188393 95.964285) (width 0.25) (layer F.Cu) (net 1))
 (segment (start 138.188393 95.964285) (end 138.433378 96.008335) (width 0.25) (layer F.Cu) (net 1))
 (segment (start 138.433378 96.008335) (end 138.677711 96.055871) (width 0.25) (layer F.Cu) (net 1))
 (segment (start 138.677711 96.055871) (end 138.921341 96.106884) (width 0.25) (layer F.Cu) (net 1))
 (segment (start 138.921341 96.106884) (end 139.164221 96.161364) (width 0.25) (layer F.Cu) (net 1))
 (segment (start 146.612345 97.431788) (end 152.34412 97.45342) (width 0.25) (layer F.Cu) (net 1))
 (segment (start 146.612345 97.431788) (end 146.363407 97.429105) (width 0.25) (layer F.Cu) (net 1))
 (segment (start 146.363407 97.429105) (end 146.114532 97.422938) (width 0.25) (layer F.Cu) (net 1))
 (segment (start 146.114532 97.422938) (end 145.865767 97.413287) (width 0.25) (layer F.Cu) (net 1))
 (segment (start 145.865767 97.413287) (end 145.617162 97.400155) (width 0.25) (layer F.Cu) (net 1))
 (segment (start 145.617162 97.400155) (end 145.368765 97.383544) (width 0.25) (layer F.Cu) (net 1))
 (segment (start 145.368765 97.383544) (end 145.120625 97.363456) (width 0.25) (layer F.Cu) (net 1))
 (segment (start 145.120625 97.363456) (end 144.872791 97.339897) (width 0.25) (layer F.Cu) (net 1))
 (segment (start 144.872791 97.339897) (end 144.625311 97.312871) (width 0.25) (layer F.Cu) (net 1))
 (segment (start 144.625311 97.312871) (end 144.378233 97.282382) (width 0.25) (layer F.Cu) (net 1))
 (segment (start 144.378233 97.282382) (end 144.131606 97.248438) (width 0.25) (layer F.Cu) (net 1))
 (segment (start 144.131606 97.248438) (end 143.885479 97.211044) (width 0.25) (layer F.Cu) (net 1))
 (segment (start 143.885479 97.211044) (end 143.639899 97.170208) (width 0.25) (layer F.Cu) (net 1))
 (segment (start 143.639899 97.170208) (end 143.394915 97.125938) (width 0.25) (layer F.Cu) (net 1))
 (segment (start 143.394915 97.125938) (end 143.150575 97.078243) (width 0.25) (layer F.Cu) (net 1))
 (segment (start 143.150575 97.078243) (end 142.906927 97.027132) (width 0.25) (layer F.Cu) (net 1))
 (segment (start 142.906927 97.027132) (end 142.664018 96.972615) (width 0.25) (layer F.Cu) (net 1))
 (segment (start 142.664018 96.972615) (end 139.164221 96.161364) (width 0.25) (layer F.Cu) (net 1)))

